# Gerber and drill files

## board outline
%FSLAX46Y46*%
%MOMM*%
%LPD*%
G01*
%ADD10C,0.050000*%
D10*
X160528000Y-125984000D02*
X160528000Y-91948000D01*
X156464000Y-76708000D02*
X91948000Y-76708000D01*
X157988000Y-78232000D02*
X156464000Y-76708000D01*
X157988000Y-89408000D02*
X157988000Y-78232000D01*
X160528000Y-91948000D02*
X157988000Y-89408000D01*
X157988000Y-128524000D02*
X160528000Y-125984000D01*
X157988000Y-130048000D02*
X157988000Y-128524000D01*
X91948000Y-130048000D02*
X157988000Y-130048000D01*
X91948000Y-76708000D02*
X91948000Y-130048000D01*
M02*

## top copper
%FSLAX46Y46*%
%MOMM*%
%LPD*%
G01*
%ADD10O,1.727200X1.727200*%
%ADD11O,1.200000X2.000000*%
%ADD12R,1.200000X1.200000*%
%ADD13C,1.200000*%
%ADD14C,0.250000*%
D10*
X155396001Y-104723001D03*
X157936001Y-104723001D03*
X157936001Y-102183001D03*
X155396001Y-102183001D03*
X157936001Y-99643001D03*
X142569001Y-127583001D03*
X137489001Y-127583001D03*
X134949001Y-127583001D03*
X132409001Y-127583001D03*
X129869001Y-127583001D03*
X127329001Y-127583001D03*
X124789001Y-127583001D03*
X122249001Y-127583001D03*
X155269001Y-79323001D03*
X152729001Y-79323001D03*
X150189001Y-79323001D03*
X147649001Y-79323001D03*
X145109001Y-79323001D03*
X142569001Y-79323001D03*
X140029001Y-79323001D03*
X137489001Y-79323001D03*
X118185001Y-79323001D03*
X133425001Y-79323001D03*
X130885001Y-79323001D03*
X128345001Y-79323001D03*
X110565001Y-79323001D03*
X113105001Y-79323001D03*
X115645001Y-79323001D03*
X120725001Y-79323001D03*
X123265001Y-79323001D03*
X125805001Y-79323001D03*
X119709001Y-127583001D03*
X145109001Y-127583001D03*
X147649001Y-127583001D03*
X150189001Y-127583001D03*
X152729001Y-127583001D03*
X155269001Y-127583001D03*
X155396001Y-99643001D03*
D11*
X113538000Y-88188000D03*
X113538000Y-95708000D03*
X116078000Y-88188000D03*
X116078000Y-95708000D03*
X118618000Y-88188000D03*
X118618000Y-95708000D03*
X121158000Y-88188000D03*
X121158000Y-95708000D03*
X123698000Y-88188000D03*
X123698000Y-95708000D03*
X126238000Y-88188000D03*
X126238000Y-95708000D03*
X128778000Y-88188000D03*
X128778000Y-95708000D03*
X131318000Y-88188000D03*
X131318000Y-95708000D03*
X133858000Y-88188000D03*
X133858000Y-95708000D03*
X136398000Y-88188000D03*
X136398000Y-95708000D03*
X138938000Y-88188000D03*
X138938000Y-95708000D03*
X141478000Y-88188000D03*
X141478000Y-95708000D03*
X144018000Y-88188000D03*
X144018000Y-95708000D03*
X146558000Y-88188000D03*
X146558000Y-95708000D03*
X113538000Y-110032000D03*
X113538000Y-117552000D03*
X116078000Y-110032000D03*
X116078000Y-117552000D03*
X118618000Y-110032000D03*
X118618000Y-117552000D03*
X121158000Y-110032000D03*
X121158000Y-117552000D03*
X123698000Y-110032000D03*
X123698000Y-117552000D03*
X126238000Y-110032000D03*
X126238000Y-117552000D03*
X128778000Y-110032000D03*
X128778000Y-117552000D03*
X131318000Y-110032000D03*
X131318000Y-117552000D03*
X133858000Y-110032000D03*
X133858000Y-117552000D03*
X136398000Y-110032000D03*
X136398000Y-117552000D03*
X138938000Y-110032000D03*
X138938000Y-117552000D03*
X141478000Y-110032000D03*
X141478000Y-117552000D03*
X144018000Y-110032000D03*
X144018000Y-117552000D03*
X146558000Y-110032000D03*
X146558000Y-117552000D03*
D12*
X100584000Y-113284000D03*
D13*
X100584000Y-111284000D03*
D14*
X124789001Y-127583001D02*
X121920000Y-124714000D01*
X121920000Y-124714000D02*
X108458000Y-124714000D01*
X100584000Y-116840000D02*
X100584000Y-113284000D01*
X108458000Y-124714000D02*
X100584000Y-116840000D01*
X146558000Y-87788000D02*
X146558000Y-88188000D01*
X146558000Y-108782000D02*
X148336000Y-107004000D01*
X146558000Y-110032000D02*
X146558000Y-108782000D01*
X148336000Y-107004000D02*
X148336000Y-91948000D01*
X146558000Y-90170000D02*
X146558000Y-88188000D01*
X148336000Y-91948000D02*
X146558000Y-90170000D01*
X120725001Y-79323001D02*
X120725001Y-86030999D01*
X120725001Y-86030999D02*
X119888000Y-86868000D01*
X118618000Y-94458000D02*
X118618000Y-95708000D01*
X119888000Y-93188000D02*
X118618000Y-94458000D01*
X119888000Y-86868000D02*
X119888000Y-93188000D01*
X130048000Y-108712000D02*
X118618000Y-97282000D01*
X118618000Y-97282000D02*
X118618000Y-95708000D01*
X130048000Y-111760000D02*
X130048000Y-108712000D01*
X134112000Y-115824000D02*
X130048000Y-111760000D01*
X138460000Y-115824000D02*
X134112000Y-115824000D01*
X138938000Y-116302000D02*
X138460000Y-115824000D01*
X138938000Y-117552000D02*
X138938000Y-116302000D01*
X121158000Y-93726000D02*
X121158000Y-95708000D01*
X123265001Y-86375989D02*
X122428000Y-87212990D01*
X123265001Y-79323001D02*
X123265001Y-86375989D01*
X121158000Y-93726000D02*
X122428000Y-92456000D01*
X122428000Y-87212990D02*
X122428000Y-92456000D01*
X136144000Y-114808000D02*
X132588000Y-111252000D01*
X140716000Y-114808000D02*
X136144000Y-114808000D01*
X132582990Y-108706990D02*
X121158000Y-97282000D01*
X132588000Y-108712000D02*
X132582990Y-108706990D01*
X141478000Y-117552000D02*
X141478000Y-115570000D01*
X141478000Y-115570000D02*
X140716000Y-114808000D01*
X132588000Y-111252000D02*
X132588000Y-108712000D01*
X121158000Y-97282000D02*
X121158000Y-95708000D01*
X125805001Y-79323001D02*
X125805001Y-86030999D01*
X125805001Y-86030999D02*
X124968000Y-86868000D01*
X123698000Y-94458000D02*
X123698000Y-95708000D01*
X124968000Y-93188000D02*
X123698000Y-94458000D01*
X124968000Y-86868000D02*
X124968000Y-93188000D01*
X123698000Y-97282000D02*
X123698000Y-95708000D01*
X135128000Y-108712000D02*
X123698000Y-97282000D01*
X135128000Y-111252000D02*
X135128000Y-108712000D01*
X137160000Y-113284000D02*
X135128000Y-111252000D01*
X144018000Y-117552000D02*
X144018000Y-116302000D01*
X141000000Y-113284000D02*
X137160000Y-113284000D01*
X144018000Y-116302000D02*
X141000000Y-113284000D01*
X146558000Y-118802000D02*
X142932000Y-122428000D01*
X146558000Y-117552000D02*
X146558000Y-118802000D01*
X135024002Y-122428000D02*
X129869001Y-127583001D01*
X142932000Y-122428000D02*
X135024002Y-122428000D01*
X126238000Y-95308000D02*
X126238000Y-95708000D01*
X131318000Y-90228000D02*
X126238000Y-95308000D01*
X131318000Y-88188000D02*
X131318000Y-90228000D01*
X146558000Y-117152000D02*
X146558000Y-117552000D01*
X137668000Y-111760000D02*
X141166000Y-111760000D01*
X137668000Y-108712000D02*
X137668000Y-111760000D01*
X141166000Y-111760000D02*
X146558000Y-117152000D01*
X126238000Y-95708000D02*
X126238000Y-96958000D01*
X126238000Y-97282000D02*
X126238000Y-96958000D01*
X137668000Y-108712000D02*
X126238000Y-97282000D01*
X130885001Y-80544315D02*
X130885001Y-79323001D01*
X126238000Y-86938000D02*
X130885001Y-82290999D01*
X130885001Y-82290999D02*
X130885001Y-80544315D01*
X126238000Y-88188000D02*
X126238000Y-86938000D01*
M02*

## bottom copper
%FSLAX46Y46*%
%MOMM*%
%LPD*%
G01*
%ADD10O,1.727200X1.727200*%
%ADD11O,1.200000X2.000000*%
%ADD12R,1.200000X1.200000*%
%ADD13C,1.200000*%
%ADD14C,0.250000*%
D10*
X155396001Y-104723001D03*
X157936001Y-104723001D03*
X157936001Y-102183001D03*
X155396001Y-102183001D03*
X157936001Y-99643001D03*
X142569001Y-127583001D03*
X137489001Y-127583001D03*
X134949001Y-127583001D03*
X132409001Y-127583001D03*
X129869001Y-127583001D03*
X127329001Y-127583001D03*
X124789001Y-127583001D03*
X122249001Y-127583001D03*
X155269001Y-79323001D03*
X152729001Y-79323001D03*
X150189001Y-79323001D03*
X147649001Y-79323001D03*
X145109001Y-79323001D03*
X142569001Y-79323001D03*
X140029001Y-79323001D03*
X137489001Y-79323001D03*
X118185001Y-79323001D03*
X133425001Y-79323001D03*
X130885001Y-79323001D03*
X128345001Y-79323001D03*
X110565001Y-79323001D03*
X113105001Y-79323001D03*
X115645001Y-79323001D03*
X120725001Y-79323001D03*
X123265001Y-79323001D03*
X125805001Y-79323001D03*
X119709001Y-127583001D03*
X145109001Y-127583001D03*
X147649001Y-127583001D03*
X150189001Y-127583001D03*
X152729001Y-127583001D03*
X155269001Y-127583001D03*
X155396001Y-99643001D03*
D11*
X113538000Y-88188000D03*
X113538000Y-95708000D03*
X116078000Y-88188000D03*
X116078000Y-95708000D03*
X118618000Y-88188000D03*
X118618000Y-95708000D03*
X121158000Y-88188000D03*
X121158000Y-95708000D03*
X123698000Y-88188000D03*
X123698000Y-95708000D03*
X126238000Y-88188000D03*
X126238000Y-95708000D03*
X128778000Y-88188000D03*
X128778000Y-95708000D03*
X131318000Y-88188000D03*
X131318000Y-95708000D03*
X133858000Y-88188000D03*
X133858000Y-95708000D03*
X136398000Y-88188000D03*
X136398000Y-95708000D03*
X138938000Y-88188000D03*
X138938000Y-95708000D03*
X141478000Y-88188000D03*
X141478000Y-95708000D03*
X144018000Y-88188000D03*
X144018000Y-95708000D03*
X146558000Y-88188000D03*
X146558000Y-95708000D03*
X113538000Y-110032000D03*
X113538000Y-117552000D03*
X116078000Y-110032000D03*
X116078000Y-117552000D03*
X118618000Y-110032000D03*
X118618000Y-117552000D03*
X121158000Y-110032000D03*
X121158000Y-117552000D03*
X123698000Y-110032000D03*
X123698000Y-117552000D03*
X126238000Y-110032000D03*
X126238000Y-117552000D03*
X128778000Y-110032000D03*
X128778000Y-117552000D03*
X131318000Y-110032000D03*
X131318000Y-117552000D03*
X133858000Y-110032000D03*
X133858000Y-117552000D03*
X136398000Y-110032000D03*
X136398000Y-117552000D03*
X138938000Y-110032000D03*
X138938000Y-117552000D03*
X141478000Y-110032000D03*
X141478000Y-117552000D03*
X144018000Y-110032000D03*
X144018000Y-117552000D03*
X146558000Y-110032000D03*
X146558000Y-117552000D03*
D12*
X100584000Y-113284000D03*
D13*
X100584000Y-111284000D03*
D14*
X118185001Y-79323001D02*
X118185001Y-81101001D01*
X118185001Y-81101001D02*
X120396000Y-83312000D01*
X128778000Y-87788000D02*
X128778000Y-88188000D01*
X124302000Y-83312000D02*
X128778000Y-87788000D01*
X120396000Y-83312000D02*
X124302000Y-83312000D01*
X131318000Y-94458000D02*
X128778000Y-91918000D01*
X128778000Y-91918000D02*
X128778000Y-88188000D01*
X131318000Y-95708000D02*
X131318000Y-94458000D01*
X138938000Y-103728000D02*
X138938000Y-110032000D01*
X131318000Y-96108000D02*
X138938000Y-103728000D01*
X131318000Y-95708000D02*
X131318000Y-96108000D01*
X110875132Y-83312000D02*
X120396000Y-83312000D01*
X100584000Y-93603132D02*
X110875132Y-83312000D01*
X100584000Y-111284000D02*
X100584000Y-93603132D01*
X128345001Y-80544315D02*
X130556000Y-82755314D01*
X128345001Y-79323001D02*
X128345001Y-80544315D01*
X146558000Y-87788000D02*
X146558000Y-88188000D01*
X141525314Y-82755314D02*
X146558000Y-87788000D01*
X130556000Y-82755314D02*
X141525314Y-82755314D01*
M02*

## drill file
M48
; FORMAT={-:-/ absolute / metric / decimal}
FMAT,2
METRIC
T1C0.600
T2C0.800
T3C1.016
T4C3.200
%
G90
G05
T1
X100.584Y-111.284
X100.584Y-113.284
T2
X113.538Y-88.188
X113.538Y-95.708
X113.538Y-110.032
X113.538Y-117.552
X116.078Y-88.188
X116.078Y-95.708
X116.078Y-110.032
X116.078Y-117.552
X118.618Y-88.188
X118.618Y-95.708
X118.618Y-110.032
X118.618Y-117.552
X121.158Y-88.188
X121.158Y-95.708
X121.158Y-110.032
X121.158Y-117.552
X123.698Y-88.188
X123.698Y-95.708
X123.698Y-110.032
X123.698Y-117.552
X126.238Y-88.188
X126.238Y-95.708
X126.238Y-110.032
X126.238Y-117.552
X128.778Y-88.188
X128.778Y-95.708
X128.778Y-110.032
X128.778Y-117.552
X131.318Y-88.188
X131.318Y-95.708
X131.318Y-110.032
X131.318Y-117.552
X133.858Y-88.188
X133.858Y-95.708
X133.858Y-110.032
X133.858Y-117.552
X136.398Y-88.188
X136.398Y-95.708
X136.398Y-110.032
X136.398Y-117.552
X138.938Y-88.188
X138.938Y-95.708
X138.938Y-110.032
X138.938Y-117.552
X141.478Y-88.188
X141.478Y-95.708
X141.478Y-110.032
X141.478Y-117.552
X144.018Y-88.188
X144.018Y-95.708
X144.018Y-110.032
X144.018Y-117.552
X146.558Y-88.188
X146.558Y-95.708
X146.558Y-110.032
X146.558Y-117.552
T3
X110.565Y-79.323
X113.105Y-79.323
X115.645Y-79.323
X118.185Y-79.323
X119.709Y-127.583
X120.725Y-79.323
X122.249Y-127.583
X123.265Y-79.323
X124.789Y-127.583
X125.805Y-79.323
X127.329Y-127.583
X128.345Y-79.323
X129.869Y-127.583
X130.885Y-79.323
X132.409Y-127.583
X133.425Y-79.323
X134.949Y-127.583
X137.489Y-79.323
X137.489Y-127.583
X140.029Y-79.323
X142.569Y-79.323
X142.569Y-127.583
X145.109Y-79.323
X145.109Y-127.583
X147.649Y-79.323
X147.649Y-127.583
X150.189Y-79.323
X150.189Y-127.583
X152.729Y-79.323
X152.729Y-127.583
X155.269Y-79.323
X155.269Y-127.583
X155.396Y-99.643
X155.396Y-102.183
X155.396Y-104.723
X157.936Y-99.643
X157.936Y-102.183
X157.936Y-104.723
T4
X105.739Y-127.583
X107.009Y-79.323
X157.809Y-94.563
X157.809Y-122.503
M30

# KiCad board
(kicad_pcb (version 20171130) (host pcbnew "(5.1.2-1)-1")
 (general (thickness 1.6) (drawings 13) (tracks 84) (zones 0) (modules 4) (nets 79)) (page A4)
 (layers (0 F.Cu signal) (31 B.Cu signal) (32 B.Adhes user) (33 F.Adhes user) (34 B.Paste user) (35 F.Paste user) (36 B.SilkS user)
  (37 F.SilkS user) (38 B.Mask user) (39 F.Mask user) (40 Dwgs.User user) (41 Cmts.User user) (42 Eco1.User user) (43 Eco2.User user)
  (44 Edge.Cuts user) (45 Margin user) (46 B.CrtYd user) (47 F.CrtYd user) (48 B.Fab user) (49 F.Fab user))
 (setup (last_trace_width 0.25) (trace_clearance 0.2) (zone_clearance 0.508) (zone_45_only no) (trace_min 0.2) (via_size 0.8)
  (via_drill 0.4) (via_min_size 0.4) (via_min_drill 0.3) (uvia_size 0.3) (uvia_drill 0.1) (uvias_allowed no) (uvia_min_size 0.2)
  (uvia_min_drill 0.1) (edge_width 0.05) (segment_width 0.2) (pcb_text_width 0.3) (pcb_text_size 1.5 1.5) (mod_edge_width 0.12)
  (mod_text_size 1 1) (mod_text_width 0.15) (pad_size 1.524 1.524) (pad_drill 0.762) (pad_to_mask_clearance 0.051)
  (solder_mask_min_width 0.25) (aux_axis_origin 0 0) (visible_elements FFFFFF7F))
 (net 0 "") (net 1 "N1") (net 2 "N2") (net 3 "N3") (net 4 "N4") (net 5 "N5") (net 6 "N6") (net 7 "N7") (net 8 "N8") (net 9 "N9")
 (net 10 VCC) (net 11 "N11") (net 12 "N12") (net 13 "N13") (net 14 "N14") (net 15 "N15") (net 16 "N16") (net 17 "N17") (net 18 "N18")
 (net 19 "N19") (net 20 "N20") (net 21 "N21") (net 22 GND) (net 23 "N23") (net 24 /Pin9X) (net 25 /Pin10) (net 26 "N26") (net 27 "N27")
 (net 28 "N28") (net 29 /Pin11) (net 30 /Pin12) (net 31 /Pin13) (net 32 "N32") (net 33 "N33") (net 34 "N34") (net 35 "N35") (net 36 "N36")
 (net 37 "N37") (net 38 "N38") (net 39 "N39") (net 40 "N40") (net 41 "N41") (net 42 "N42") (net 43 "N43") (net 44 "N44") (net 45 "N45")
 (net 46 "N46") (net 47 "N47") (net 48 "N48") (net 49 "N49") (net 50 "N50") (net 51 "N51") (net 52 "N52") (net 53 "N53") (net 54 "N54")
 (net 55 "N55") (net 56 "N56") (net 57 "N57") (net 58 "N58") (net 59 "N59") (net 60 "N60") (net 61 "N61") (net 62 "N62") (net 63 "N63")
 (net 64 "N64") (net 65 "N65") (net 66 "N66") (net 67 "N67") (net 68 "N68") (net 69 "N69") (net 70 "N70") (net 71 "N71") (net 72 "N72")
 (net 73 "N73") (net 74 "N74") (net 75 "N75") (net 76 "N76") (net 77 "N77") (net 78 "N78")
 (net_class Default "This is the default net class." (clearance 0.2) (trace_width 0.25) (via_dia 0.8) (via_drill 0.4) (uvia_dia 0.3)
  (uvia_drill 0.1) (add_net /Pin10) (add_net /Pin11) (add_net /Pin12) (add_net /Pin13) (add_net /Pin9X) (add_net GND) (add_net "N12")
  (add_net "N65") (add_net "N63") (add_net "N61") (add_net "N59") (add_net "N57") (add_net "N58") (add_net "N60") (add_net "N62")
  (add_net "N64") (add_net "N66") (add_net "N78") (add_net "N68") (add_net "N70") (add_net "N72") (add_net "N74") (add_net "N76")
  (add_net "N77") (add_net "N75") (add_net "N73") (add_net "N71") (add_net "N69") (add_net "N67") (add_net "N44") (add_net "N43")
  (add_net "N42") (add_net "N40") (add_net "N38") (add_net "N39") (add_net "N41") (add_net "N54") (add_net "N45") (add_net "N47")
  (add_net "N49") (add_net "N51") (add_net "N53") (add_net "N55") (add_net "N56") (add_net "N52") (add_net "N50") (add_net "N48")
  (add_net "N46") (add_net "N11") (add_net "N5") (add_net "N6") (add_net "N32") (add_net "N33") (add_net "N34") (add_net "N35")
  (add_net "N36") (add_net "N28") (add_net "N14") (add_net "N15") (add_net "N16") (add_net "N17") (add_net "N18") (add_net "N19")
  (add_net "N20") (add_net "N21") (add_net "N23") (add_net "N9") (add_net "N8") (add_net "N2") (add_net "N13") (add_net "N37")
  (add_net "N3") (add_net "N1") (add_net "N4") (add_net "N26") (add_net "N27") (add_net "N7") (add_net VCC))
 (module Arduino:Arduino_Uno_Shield (layer F.Cu) (at 91.769001 130.123001)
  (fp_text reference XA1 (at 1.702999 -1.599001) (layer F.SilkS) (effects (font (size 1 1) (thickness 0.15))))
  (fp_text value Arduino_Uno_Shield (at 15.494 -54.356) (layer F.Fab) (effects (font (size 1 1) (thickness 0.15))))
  (pad RST2 thru_hole oval (at 63.627 -25.4) (size 1.7272 1.7272) (drill 1.016) (layers *.Cu *.Mask) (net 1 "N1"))
  (pad GND4 thru_hole oval (at 66.167 -25.4) (size 1.7272 1.7272) (drill 1.016) (layers *.Cu *.Mask) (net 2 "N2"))
  (pad MOSI thru_hole oval (at 66.167 -27.94) (size 1.7272 1.7272) (drill 1.016) (layers *.Cu *.Mask) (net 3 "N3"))
  (pad SCK thru_hole oval (at 63.627 -27.94) (size 1.7272 1.7272) (drill 1.016) (layers *.Cu *.Mask) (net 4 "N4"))
  (pad 5V2 thru_hole oval (at 66.167 -30.48) (size 1.7272 1.7272) (drill 1.016) (layers *.Cu *.Mask) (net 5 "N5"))
  (pad A0 thru_hole oval (at 50.8 -2.54) (size 1.7272 1.7272) (drill 1.016) (layers *.Cu *.Mask) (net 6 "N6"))
  (pad VIN thru_hole oval (at 45.72 -2.54) (size 1.7272 1.7272) (drill 1.016) (layers *.Cu *.Mask) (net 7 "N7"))
  (pad GND3 thru_hole oval (at 43.18 -2.54) (size 1.7272 1.7272) (drill 1.016) (layers *.Cu *.Mask) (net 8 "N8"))
  (pad GND2 thru_hole oval (at 40.64 -2.54) (size 1.7272 1.7272) (drill 1.016) (layers *.Cu *.Mask) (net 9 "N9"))
  (pad 5V1 thru_hole oval (at 38.1 -2.54) (size 1.7272 1.7272) (drill 1.016) (layers *.Cu *.Mask) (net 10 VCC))
  (pad 3V3 thru_hole oval (at 35.56 -2.54) (size 1.7272 1.7272) (drill 1.016) (layers *.Cu *.Mask) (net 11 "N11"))
  (pad RST1 thru_hole oval (at 33.02 -2.54) (size 1.7272 1.7272) (drill 1.016) (layers *.Cu *.Mask) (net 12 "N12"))
  (pad IORF thru_hole oval (at 30.48 -2.54) (size 1.7272 1.7272) (drill 1.016) (layers *.Cu *.Mask) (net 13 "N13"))
  (pad D0 thru_hole oval (at 63.5 -50.8) (size 1.7272 1.7272) (drill 1.016) (layers *.Cu *.Mask) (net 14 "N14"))
  (pad D1 thru_hole oval (at 60.96 -50.8) (size 1.7272 1.7272) (drill 1.016) (layers *.Cu *.Mask) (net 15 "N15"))
  (pad D2 thru_hole oval (at 58.42 -50.8) (size 1.7272 1.7272) (drill 1.016) (layers *.Cu *.Mask) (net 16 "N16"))
  (pad D3 thru_hole oval (at 55.88 -50.8) (size 1.7272 1.7272) (drill 1.016) (layers *.Cu *.Mask) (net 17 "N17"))
  (pad D4 thru_hole oval (at 53.34 -50.8) (size 1.7272 1.7272) (drill 1.016) (layers *.Cu *.Mask) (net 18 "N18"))
  (pad D5 thru_hole oval (at 50.8 -50.8) (size 1.7272 1.7272) (drill 1.016) (layers *.Cu *.Mask) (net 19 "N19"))
  (pad D6 thru_hole oval (at 48.26 -50.8) (size 1.7272 1.7272) (drill 1.016) (layers *.Cu *.Mask) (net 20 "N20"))
  (pad D7 thru_hole oval (at 45.72 -50.8) (size 1.7272 1.7272) (drill 1.016) (layers *.Cu *.Mask) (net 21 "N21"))
  (pad GND1 thru_hole oval (at 26.416 -50.8) (size 1.7272 1.7272) (drill 1.016) (layers *.Cu *.Mask) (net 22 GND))
  (pad D8 thru_hole oval (at 41.656 -50.8) (size 1.7272 1.7272) (drill 1.016) (layers *.Cu *.Mask) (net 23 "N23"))
  (pad D9 thru_hole oval (at 39.116 -50.8) (size 1.7272 1.7272) (drill 1.016) (layers *.Cu *.Mask) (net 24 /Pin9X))
  (pad D10 thru_hole oval (at 36.576 -50.8) (size 1.7272 1.7272) (drill 1.016) (layers *.Cu *.Mask) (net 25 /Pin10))
  (pad "" np_thru_hole circle (at 66.04 -7.62) (size 3.2 3.2) (drill 3.2) (layers *.Cu *.Mask))
  (pad "" np_thru_hole circle (at 66.04 -35.56) (size 3.2 3.2) (drill 3.2) (layers *.Cu *.Mask))
  (pad "" np_thru_hole circle (at 15.24 -50.8) (size 3.2 3.2) (drill 3.2) (layers *.Cu *.Mask))
  (pad "" np_thru_hole circle (at 13.97 -2.54) (size 3.2 3.2) (drill 3.2) (layers *.Cu *.Mask))
  (pad SCL thru_hole oval (at 18.796 -50.8) (size 1.7272 1.7272) (drill 1.016) (layers *.Cu *.Mask) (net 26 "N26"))
  (pad SDA thru_hole oval (at 21.336 -50.8) (size 1.7272 1.7272) (drill 1.016) (layers *.Cu *.Mask) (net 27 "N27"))
  (pad AREF thru_hole oval (at 23.876 -50.8) (size 1.7272 1.7272) (drill 1.016) (layers *.Cu *.Mask) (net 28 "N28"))
  (pad D13 thru_hole oval (at 28.956 -50.8) (size 1.7272 1.7272) (drill 1.016) (layers *.Cu *.Mask) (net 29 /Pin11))
  (pad D12 thru_hole oval (at 31.496 -50.8) (size 1.7272 1.7272) (drill 1.016) (layers *.Cu *.Mask) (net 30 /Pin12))
  (pad D11 thru_hole oval (at 34.036 -50.8) (size 1.7272 1.7272) (drill 1.016) (layers *.Cu *.Mask) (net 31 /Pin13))
  (pad "" thru_hole oval (at 27.94 -2.54) (size 1.7272 1.7272) (drill 1.016) (layers *.Cu *.Mask))
  (pad A1 thru_hole oval (at 53.34 -2.54) (size 1.7272 1.7272) (drill 1.016) (layers *.Cu *.Mask) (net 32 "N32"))
  (pad A2 thru_hole oval (at 55.88 -2.54) (size 1.7272 1.7272) (drill 1.016) (layers *.Cu *.Mask) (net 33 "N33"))
  (pad A3 thru_hole oval (at 58.42 -2.54) (size 1.7272 1.7272) (drill 1.016) (layers *.Cu *.Mask) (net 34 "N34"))
  (pad A4 thru_hole oval (at 60.96 -2.54) (size 1.7272 1.7272) (drill 1.016) (layers *.Cu *.Mask) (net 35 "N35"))
  (pad A5 thru_hole oval (at 63.5 -2.54) (size 1.7272 1.7272) (drill 1.016) (layers *.Cu *.Mask) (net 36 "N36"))
  (pad MISO thru_hole oval (at 63.627 -30.48) (size 1.7272 1.7272) (drill 1.016) (layers *.Cu *.Mask) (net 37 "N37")))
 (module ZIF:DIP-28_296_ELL (layer F.Cu) (at 130.048 91.948 180)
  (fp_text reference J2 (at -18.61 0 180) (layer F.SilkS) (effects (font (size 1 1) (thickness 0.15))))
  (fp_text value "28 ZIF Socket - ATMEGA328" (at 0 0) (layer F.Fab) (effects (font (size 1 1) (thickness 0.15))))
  (pad 14 thru_hole oval (at 16.51 3.76 180) (size 1.2 2) (drill 0.8) (layers *.Cu *.Mask) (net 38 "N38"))
  (pad 15 thru_hole oval (at 16.51 -3.76 180) (size 1.2 2) (drill 0.8) (layers *.Cu *.Mask) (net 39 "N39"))
  (pad 13 thru_hole oval (at 13.97 3.76 180) (size 1.2 2) (drill 0.8) (layers *.Cu *.Mask) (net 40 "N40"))
  (pad 16 thru_hole oval (at 13.97 -3.76 180) (size 1.2 2) (drill 0.8) (layers *.Cu *.Mask) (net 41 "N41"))
  (pad 12 thru_hole oval (at 11.43 3.76 180) (size 1.2 2) (drill 0.8) (layers *.Cu *.Mask) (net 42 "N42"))
  (pad 17 thru_hole oval (at 11.43 -3.76 180) (size 1.2 2) (drill 0.8) (layers *.Cu *.Mask) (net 29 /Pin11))
  (pad 11 thru_hole oval (at 8.89 3.76 180) (size 1.2 2) (drill 0.8) (layers *.Cu *.Mask) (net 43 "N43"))
  (pad 18 thru_hole oval (at 8.89 -3.76 180) (size 1.2 2) (drill 0.8) (layers *.Cu *.Mask) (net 30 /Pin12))
  (pad 10 thru_hole oval (at 6.35 3.76 180) (size 1.2 2) (drill 0.8) (layers *.Cu *.Mask) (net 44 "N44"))
  (pad 19 thru_hole oval (at 6.35 -3.76 180) (size 1.2 2) (drill 0.8) (layers *.Cu *.Mask) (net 31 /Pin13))
  (pad 9 thru_hole oval (at 3.81 3.76 180) (size 1.2 2) (drill 0.8) (layers *.Cu *.Mask) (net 24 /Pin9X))
  (pad 20 thru_hole oval (at 3.81 -3.76 180) (size 1.2 2) (drill 0.8) (layers *.Cu *.Mask) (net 10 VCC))
  (pad 8 thru_hole oval (at 1.27 3.76 180) (size 1.2 2) (drill 0.8) (layers *.Cu *.Mask) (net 22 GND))
  (pad 21 thru_hole oval (at 1.27 -3.76 180) (size 1.2 2) (drill 0.8) (layers *.Cu *.Mask) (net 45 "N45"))
  (pad 7 thru_hole oval (at -1.27 3.76 180) (size 1.2 2) (drill 0.8) (layers *.Cu *.Mask) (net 10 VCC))
  (pad 22 thru_hole oval (at -1.27 -3.76 180) (size 1.2 2) (drill 0.8) (layers *.Cu *.Mask) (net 22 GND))
  (pad 6 thru_hole oval (at -3.81 3.76 180) (size 1.2 2) (drill 0.8) (layers *.Cu *.Mask) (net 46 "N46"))
  (pad 23 thru_hole oval (at -3.81 -3.76 180) (size 1.2 2) (drill 0.8) (layers *.Cu *.Mask) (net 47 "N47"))
  (pad 5 thru_hole oval (at -6.35 3.76 180) (size 1.2 2) (drill 0.8) (layers *.Cu *.Mask) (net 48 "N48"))
  (pad 24 thru_hole oval (at -6.35 -3.76 180) (size 1.2 2) (drill 0.8) (layers *.Cu *.Mask) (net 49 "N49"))
  (pad 4 thru_hole oval (at -8.89 3.76 180) (size 1.2 2) (drill 0.8) (layers *.Cu *.Mask) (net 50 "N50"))
  (pad 25 thru_hole oval (at -8.89 -3.76 180) (size 1.2 2) (drill 0.8) (layers *.Cu *.Mask) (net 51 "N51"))
  (pad 3 thru_hole oval (at -11.43 3.76 180) (size 1.2 2) (drill 0.8) (layers *.Cu *.Mask) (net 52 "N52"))
  (pad 26 thru_hole oval (at -11.43 -3.76 180) (size 1.2 2) (drill 0.8) (layers *.Cu *.Mask) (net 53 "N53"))
  (pad 2 thru_hole oval (at -13.97 3.76 180) (size 1.2 2) (drill 0.8) (layers *.Cu *.Mask) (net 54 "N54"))
  (pad 27 thru_hole oval (at -13.97 -3.76 180) (size 1.2 2) (drill 0.8) (layers *.Cu *.Mask) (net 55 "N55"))
  (pad 1 thru_hole oval (at -16.51 3.76 180) (size 1.2 2) (drill 0.8) (layers *.Cu *.Mask) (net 25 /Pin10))
  (pad 28 thru_hole oval (at -16.51 -3.76 180) (size 1.2 2) (drill 0.8) (layers *.Cu *.Mask) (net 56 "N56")))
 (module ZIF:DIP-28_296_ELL (layer F.Cu) (at 130.048 113.792 180)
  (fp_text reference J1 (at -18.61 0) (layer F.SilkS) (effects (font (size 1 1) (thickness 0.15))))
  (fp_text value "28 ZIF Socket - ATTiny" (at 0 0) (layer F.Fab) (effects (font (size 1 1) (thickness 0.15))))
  (pad 14 thru_hole oval (at 16.51 3.76 180) (size 1.2 2) (drill 0.8) (layers *.Cu *.Mask) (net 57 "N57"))
  (pad 15 thru_hole oval (at 16.51 -3.76 180) (size 1.2 2) (drill 0.8) (layers *.Cu *.Mask) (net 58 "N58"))
  (pad 13 thru_hole oval (at 13.97 3.76 180) (size 1.2 2) (drill 0.8) (layers *.Cu *.Mask) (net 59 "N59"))
  (pad 16 thru_hole oval (at 13.97 -3.76 180) (size 1.2 2) (drill 0.8) (layers *.Cu *.Mask) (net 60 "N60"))
  (pad 12 thru_hole oval (at 11.43 3.76 180) (size 1.2 2) (drill 0.8) (layers *.Cu *.Mask) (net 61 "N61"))
  (pad 17 thru_hole oval (at 11.43 -3.76 180) (size 1.2 2) (drill 0.8) (layers *.Cu *.Mask) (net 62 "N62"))
  (pad 11 thru_hole oval (at 8.89 3.76 180) (size 1.2 2) (drill 0.8) (layers *.Cu *.Mask) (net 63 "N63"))
  (pad 18 thru_hole oval (at 8.89 -3.76 180) (size 1.2 2) (drill 0.8) (layers *.Cu *.Mask) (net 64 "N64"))
  (pad 10 thru_hole oval (at 6.35 3.76 180) (size 1.2 2) (drill 0.8) (layers *.Cu *.Mask) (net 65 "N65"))
  (pad 19 thru_hole oval (at 6.35 -3.76 180) (size 1.2 2) (drill 0.8) (layers *.Cu *.Mask) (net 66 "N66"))
  (pad 9 thru_hole oval (at 3.81 3.76 180) (size 1.2 2) (drill 0.8) (layers *.Cu *.Mask) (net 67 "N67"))
  (pad 20 thru_hole oval (at 3.81 -3.76 180) (size 1.2 2) (drill 0.8) (layers *.Cu *.Mask) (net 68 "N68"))
  (pad 8 thru_hole oval (at 1.27 3.76 180) (size 1.2 2) (drill 0.8) (layers *.Cu *.Mask) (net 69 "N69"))
  (pad 21 thru_hole oval (at 1.27 -3.76 180) (size 1.2 2) (drill 0.8) (layers *.Cu *.Mask) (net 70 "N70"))
  (pad 7 thru_hole oval (at -1.27 3.76 180) (size 1.2 2) (drill 0.8) (layers *.Cu *.Mask) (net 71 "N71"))
  (pad 22 thru_hole oval (at -1.27 -3.76 180) (size 1.2 2) (drill 0.8) (layers *.Cu *.Mask) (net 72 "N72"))
  (pad 6 thru_hole oval (at -3.81 3.76 180) (size 1.2 2) (drill 0.8) (layers *.Cu *.Mask) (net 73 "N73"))
  (pad 23 thru_hole oval (at -3.81 -3.76 180) (size 1.2 2) (drill 0.8) (layers *.Cu *.Mask) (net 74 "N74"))
  (pad 5 thru_hole oval (at -6.35 3.76 180) (size 1.2 2) (drill 0.8) (layers *.Cu *.Mask) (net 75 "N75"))
  (pad 24 thru_hole oval (at -6.35 -3.76 180) (size 1.2 2) (drill 0.8) (layers *.Cu *.Mask) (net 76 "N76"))
  (pad 4 thru_hole oval (at -8.89 3.76 180) (size 1.2 2) (drill 0.8) (layers *.Cu *.Mask) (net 22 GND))
  (pad 25 thru_hole oval (at -8.89 -3.76 180) (size 1.2 2) (drill 0.8) (layers *.Cu *.Mask) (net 29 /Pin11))
  (pad 3 thru_hole oval (at -11.43 3.76 180) (size 1.2 2) (drill 0.8) (layers *.Cu *.Mask) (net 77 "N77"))
  (pad 26 thru_hole oval (at -11.43 -3.76 180) (size 1.2 2) (drill 0.8) (layers *.Cu *.Mask) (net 30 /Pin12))
  (pad 2 thru_hole oval (at -13.97 3.76 180) (size 1.2 2) (drill 0.8) (layers *.Cu *.Mask) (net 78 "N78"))
  (pad 27 thru_hole oval (at -13.97 -3.76 180) (size 1.2 2) (drill 0.8) (layers *.Cu *.Mask) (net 31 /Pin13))
  (pad 1 thru_hole oval (at -16.51 3.76 180) (size 1.2 2) (drill 0.8) (layers *.Cu *.Mask) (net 25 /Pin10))
  (pad 28 thru_hole oval (at -16.51 -3.76 180) (size 1.2 2) (drill 0.8) (layers *.Cu *.Mask) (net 10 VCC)))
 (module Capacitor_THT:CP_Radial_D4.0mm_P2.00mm (layer F.Cu) (at 100.584 113.284 90)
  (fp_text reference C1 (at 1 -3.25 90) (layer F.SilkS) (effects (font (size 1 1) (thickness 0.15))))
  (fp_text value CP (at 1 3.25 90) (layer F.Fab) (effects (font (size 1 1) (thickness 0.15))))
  (pad 1 thru_hole rect (at 0 0 90) (size 1.2 1.2) (drill 0.6) (layers *.Cu *.Mask) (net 12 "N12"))
  (pad 2 thru_hole circle (at 2 0 90) (size 1.2 1.2) (drill 0.6) (layers *.Cu *.Mask) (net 22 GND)))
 (gr_line (start 160.528 125.984) (end 160.528 91.948) (layer Edge.Cuts) (width 0.05))
 (gr_line (start 156.464 76.708) (end 91.948 76.708) (layer Edge.Cuts) (width 0.05))
 (gr_line (start 157.988 78.232) (end 156.464 76.708) (layer Edge.Cuts) (width 0.05))
 (gr_line (start 157.988 89.408) (end 157.988 78.232) (layer Edge.Cuts) (width 0.05))
 (gr_line (start 160.528 91.948) (end 157.988 89.408) (layer Edge.Cuts) (width 0.05))
 (gr_line (start 157.988 128.524) (end 160.528 125.984) (layer Edge.Cuts) (width 0.05))
 (gr_line (start 157.988 130.048) (end 157.988 128.524) (layer Edge.Cuts) (width 0.05))
 (gr_line (start 91.948 130.048) (end 157.988 130.048) (layer Edge.Cuts) (width 0.05))
 (gr_line (start 91.948 76.708) (end 91.948 130.048) (layer Edge.Cuts) (width 0.05))
 (segment (start 124.789001 127.583001) (end 121.92 124.714) (width 0.25) (layer F.Cu) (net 12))
 (segment (start 121.92 124.714) (end 108.458 124.714) (width 0.25) (layer F.Cu) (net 12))
 (segment (start 100.584 116.84) (end 100.584 113.284) (width 0.25) (layer F.Cu) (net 12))
 (segment (start 108.458 124.714) (end 100.584 116.84) (width 0.25) (layer F.Cu) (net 12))
 (segment (start 118.185001 79.323001) (end 118.185001 81.101001) (width 0.25) (layer B.Cu) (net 22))
 (segment (start 118.185001 81.101001) (end 120.396 83.312) (width 0.25) (layer B.Cu) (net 22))
 (segment (start 128.778 87.788) (end 128.778 88.188) (width 0.25) (layer B.Cu) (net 22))
 (segment (start 124.302 83.312) (end 128.778 87.788) (width 0.25) (layer B.Cu) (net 22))
 (segment (start 120.396 83.312) (end 124.302 83.312) (width 0.25) (layer B.Cu) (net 22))
 (segment (start 131.318 94.458) (end 128.778 91.918) (width 0.25) (layer B.Cu) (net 22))
 (segment (start 128.778 91.918) (end 128.778 88.188) (width 0.25) (layer B.Cu) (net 22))
 (segment (start 131.318 95.708) (end 131.318 94.458) (width 0.25) (layer B.Cu) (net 22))
 (segment (start 138.938 103.728) (end 138.938 110.032) (width 0.25) (layer B.Cu) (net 22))
 (segment (start 131.318 96.108) (end 138.938 103.728) (width 0.25) (layer B.Cu) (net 22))
 (segment (start 131.318 95.708) (end 131.318 96.108) (width 0.25) (layer B.Cu) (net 22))
 (segment (start 110.875132 83.312) (end 120.396 83.312) (width 0.25) (layer B.Cu) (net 22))
 (segment (start 100.584 93.603132) (end 110.875132 83.312) (width 0.25) (layer B.Cu) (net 22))
 (segment (start 100.584 111.284) (end 100.584 93.603132) (width 0.25) (layer B.Cu) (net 22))
 (segment (start 146.558 87.788) (end 146.558 88.188) (width 0.25) (layer F.Cu) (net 25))
 (segment (start 146.558 108.782) (end 148.336 107.004) (width 0.25) (layer F.Cu) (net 25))
 (segment (start 146.558 110.032) (end 146.558 108.782) (width 0.25) (layer F.Cu) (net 25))
 (segment (start 148.336 107.004) (end 148.336 91.948) (width 0.25) (layer F.Cu) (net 25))
 (segment (start 146.558 90.17) (end 146.558 88.188) (width 0.25) (layer F.Cu) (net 25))
 (segment (start 148.336 91.948) (end 146.558 90.17) (width 0.25) (layer F.Cu) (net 25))
 (segment (start 128.345001 80.544315) (end 130.556 82.755314) (width 0.25) (layer B.Cu) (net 25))
 (segment (start 128.345001 79.323001) (end 128.345001 80.544315) (width 0.25) (layer B.Cu) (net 25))
 (segment (start 146.558 87.788) (end 146.558 88.188) (width 0.25) (layer B.Cu) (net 25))
 (segment (start 141.525314 82.755314) (end 146.558 87.788) (width 0.25) (layer B.Cu) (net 25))
 (segment (start 130.556 82.755314) (end 141.525314 82.755314) (width 0.25) (layer B.Cu) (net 25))
 (segment (start 120.725001 79.323001) (end 120.725001 86.030999) (width 0.25) (layer F.Cu) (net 29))
 (segment (start 120.725001 86.030999) (end 119.888 86.868) (width 0.25) (layer F.Cu) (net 29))
 (segment (start 118.618 94.458) (end 118.618 95.708) (width 0.25) (layer F.Cu) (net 29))
 (segment (start 119.888 93.188) (end 118.618 94.458) (width 0.25) (layer F.Cu) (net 29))
 (segment (start 119.888 86.868) (end 119.888 93.188) (width 0.25) (layer F.Cu) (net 29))
 (segment (start 130.048 108.712) (end 118.618 97.282) (width 0.25) (layer F.Cu) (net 29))
 (segment (start 118.618 97.282) (end 118.618 95.708) (width 0.25) (layer F.Cu) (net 29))
 (segment (start 130.048 111.76) (end 130.048 108.712) (width 0.25) (layer F.Cu) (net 29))
 (segment (start 134.112 115.824) (end 130.048 111.76) (width 0.25) (layer F.Cu) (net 29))
 (segment (start 138.46 115.824) (end 134.112 115.824) (width 0.25) (layer F.Cu) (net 29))
 (segment (start 138.938 116.302) (end 138.46 115.824) (width 0.25) (layer F.Cu) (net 29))
 (segment (start 138.938 117.552) (end 138.938 116.302) (width 0.25) (layer F.Cu) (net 29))
 (segment (start 121.158 93.726) (end 121.158 95.708) (width 0.25) (layer F.Cu) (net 30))
 (segment (start 123.265001 86.375989) (end 122.428 87.21299) (width 0.25) (layer F.Cu) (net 30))
 (segment (start 123.265001 79.323001) (end 123.265001 86.375989) (width 0.25) (layer F.Cu) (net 30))
 (segment (start 121.158 93.726) (end 122.428 92.456) (width 0.25) (layer F.Cu) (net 30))
 (segment (start 122.428 87.21299) (end 122.428 92.456) (width 0.25) (layer F.Cu) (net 30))
 (segment (start 136.144 114.808) (end 132.588 111.252) (width 0.25) (layer F.Cu) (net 30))
 (segment (start 140.716 114.808) (end 136.144 114.808) (width 0.25) (layer F.Cu) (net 30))
 (segment (start 132.58299 108.70699) (end 121.158 97.282) (width 0.25) (layer F.Cu) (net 30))
 (segment (start 132.588 108.712) (end 132.58299 108.70699) (width 0.25) (layer F.Cu) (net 30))
 (segment (start 141.478 117.552) (end 141.478 115.57) (width 0.25) (layer F.Cu) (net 30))
 (segment (start 141.478 115.57) (end 140.716 114.808) (width 0.25) (layer F.Cu) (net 30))
 (segment (start 132.588 111.252) (end 132.588 108.712) (width 0.25) (layer F.Cu) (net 30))
 (segment (start 121.158 97.282) (end 121.158 95.708) (width 0.25) (layer F.Cu) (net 30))
 (segment (start 125.805001 79.323001) (end 125.805001 86.030999) (width 0.25) (layer F.Cu) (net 31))
 (segment (start 125.805001 86.030999) (end 124.968 86.868) (width 0.25) (layer F.Cu) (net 31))
 (segment (start 123.698 94.458) (end 123.698 95.708) (width 0.25) (layer F.Cu) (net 31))
 (segment (start 124.968 93.188) (end 123.698 94.458) (width 0.25) (layer F.Cu) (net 31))
 (segment (start 124.968 86.868) (end 124.968 93.188) (width 0.25) (layer F.Cu) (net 31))
 (segment (start 123.698 97.282) (end 123.698 95.708) (width 0.25) (layer F.Cu) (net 31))
 (segment (start 135.128 108.712) (end 123.698 97.282) (width 0.25) (layer F.Cu) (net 31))
 (segment (start 135.128 111.252) (end 135.128 108.712) (width 0.25) (layer F.Cu) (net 31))
 (segment (start 137.16 113.284) (end 135.128 111.252) (width 0.25) (layer F.Cu) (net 31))
 (segment (start 144.018 117.552) (end 144.018 116.302) (width 0.25) (layer F.Cu) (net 31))
 (segment (start 141 113.284) (end 137.16 113.284) (width 0.25) (layer F.Cu) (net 31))
 (segment (start 144.018 116.302) (end 141 113.284) (width 0.25) (layer F.Cu) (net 31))
 (segment (start 146.558 118.802) (end 142.932 122.428) (width 0.25) (layer F.Cu) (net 10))
 (segment (start 146.558 117.552) (end 146.558 118.802) (width 0.25) (layer F.Cu) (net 10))
 (segment (start 135.024002 122.428) (end 129.869001 127.583001) (width 0.25) (layer F.Cu) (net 10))
 (segment (start 142.932 122.428) (end 135.024002 122.428) (width 0.25) (layer F.Cu) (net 10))
 (segment (start 126.238 95.308) (end 126.238 95.708) (width 0.25) (layer F.Cu) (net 10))
 (segment (start 131.318 90.228) (end 126.238 95.308) (width 0.25) (layer F.Cu) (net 10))
 (segment (start 131.318 88.188) (end 131.318 90.228) (width 0.25) (layer F.Cu) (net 10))
 (segment (start 146.558 117.152) (end 146.558 117.552) (width 0.25) (layer F.Cu) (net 10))
 (segment (start 137.668 111.76) (end 141.166 111.76) (width 0.25) (layer F.Cu) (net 10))
 (segment (start 137.668 108.712) (end 137.668 111.76) (width 0.25) (layer F.Cu) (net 10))
 (segment (start 141.166 111.76) (end 146.558 117.152) (width 0.25) (layer F.Cu) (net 10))
 (segment (start 126.238 95.708) (end 126.238 96.958) (width 0.25) (layer F.Cu) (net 10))
 (segment (start 126.238 97.282) (end 126.238 96.958) (width 0.25) (layer F.Cu) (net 10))
 (segment (start 137.668 108.712) (end 126.238 97.282) (width 0.25) (layer F.Cu) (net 10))
 (segment (start 130.885001 80.544315) (end 130.885001 79.323001) (width 0.25) (layer F.Cu) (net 24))
 (segment (start 126.238 86.938) (end 130.885001 82.290999) (width 0.25) (layer F.Cu) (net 24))
 (segment (start 130.885001 82.290999) (end 130.885001 80.544315) (width 0.25) (layer F.Cu) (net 24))
 (segment (start 126.238 88.188) (end 126.238 86.938) (width 0.25) (layer F.Cu) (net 24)))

